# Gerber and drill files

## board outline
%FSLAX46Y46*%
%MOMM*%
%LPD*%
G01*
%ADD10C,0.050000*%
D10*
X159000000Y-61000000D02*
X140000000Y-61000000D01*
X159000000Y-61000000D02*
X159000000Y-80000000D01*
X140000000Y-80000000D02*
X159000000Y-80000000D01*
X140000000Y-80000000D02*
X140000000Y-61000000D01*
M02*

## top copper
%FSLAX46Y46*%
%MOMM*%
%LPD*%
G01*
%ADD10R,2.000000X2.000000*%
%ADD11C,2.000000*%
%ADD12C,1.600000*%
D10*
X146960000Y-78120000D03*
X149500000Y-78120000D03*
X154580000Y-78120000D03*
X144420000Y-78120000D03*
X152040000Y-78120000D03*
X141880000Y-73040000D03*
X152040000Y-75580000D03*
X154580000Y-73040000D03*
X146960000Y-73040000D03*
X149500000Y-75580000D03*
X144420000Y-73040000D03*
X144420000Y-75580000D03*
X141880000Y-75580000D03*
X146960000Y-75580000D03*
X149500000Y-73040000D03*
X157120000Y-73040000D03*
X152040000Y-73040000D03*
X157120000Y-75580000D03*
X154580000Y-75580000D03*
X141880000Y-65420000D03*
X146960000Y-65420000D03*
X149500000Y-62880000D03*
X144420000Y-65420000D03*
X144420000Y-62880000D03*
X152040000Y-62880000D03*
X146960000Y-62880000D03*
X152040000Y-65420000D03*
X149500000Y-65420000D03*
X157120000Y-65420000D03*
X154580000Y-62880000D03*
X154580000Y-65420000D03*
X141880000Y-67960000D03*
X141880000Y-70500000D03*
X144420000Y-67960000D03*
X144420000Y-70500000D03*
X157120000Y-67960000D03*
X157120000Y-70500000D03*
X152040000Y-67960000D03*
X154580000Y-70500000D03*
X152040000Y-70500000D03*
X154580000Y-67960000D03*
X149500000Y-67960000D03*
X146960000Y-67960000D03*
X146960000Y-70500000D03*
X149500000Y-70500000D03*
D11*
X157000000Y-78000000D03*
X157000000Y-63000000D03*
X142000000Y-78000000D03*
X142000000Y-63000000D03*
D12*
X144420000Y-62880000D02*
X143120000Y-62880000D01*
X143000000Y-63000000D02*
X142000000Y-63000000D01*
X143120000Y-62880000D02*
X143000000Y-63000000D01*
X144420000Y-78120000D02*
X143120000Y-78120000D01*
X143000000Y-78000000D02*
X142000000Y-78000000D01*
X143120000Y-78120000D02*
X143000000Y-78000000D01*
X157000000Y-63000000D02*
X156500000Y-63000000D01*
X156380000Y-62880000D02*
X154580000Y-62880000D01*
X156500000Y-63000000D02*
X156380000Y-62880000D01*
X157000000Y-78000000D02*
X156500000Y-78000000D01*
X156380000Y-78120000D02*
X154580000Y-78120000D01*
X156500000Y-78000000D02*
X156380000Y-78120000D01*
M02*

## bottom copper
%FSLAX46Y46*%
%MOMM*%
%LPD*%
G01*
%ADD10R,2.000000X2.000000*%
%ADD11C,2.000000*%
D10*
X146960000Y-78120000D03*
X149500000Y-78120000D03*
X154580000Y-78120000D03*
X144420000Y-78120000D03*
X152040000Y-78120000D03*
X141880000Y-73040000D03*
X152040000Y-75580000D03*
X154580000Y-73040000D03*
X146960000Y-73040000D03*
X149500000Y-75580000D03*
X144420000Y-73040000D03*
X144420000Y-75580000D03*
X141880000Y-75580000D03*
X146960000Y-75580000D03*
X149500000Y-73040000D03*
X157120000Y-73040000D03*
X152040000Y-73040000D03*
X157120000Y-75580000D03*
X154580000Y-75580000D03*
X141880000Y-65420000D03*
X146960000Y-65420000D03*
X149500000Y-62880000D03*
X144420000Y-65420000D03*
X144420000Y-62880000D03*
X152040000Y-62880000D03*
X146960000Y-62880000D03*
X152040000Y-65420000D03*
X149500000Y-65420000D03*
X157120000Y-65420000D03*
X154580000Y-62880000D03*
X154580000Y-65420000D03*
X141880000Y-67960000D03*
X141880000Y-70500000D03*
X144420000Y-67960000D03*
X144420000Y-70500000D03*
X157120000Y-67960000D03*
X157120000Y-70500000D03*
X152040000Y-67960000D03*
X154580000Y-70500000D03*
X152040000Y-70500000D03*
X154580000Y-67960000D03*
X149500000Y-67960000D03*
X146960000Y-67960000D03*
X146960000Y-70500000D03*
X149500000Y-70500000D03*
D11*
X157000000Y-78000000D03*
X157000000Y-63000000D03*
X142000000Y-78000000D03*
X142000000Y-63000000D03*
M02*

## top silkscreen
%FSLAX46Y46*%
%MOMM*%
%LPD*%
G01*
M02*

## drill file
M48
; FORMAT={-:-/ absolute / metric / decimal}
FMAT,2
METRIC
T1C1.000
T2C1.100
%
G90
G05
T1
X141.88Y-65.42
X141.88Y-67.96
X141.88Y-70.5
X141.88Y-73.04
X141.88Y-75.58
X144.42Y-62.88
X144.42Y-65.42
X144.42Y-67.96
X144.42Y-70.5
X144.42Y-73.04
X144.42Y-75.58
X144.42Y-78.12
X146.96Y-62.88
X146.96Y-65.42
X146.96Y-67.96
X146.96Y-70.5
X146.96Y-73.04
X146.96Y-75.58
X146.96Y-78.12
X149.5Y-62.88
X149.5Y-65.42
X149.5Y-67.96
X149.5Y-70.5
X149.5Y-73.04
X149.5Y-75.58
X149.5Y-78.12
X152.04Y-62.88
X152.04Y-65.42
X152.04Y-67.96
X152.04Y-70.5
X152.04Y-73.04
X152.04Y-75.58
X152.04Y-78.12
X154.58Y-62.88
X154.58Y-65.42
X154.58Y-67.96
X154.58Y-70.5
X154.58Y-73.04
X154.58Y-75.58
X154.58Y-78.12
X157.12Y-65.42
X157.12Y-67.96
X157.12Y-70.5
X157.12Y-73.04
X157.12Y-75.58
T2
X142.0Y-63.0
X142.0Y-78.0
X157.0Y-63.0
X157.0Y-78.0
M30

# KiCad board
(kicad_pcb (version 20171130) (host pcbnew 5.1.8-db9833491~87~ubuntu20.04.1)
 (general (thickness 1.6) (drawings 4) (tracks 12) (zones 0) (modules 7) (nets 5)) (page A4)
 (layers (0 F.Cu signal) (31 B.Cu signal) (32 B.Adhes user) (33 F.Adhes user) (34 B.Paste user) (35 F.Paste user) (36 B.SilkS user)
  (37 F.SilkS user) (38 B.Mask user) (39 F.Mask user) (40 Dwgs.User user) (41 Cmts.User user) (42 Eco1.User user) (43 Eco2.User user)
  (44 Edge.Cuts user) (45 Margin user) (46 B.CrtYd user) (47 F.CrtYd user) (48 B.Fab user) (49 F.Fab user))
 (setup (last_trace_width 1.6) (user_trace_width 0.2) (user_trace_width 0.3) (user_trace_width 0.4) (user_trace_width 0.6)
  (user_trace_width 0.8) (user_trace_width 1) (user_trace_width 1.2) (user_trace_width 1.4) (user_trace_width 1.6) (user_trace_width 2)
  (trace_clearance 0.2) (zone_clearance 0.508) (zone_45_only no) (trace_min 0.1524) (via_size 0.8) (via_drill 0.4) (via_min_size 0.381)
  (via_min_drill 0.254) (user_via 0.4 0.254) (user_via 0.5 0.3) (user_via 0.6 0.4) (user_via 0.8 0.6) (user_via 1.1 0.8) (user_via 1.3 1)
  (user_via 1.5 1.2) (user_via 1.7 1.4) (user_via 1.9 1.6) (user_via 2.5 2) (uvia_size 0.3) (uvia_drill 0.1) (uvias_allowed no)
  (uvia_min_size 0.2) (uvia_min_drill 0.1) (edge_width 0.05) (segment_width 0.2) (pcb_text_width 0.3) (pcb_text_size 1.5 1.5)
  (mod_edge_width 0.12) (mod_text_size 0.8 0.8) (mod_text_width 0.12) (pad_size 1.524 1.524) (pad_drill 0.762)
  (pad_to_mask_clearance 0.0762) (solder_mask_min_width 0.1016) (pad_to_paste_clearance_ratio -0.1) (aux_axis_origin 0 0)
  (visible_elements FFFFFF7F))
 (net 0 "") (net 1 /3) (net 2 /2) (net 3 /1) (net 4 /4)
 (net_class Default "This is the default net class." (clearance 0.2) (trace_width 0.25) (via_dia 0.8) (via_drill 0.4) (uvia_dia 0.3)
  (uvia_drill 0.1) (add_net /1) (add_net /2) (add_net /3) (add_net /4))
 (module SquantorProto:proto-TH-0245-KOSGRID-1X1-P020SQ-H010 (layer F.Cu) (at 149.5 70.5)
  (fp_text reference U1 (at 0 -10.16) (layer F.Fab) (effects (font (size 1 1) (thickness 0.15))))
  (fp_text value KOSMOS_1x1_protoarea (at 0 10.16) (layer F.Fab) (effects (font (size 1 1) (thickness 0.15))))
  (pad NC thru_hole rect (at -2.54 7.62) (size 2 2) (drill 1) (layers *.Cu *.Mask))
  (pad NC thru_hole rect (at 0 7.62) (size 2 2) (drill 1) (layers *.Cu *.Mask))
  (pad 3 thru_hole rect (at 5.08 7.62) (size 2 2) (drill 1) (layers *.Cu *.Mask) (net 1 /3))
  (pad 2 thru_hole rect (at -5.08 7.62) (size 2 2) (drill 1) (layers *.Cu *.Mask) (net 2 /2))
  (pad NC thru_hole rect (at 2.54 7.62) (size 2 2) (drill 1) (layers *.Cu *.Mask))
  (pad NC thru_hole rect (at -7.62 2.54) (size 2 2) (drill 1) (layers *.Cu *.Mask))
  (pad NC thru_hole rect (at 2.54 5.08) (size 2 2) (drill 1) (layers *.Cu *.Mask))
  (pad NC thru_hole rect (at 5.08 2.54) (size 2 2) (drill 1) (layers *.Cu *.Mask))
  (pad NC thru_hole rect (at -2.54 2.54) (size 2 2) (drill 1) (layers *.Cu *.Mask))
  (pad NC thru_hole rect (at 0 5.08) (size 2 2) (drill 1) (layers *.Cu *.Mask))
  (pad NC thru_hole rect (at -5.08 2.54) (size 2 2) (drill 1) (layers *.Cu *.Mask))
  (pad NC thru_hole rect (at -5.08 5.08) (size 2 2) (drill 1) (layers *.Cu *.Mask))
  (pad NC thru_hole rect (at -7.62 5.08) (size 2 2) (drill 1) (layers *.Cu *.Mask))
  (pad NC thru_hole rect (at -2.54 5.08) (size 2 2) (drill 1) (layers *.Cu *.Mask))
  (pad NC thru_hole rect (at 0 2.54) (size 2 2) (drill 1) (layers *.Cu *.Mask))
  (pad NC thru_hole rect (at 7.62 2.54) (size 2 2) (drill 1) (layers *.Cu *.Mask))
  (pad NC thru_hole rect (at 2.54 2.54) (size 2 2) (drill 1) (layers *.Cu *.Mask))
  (pad NC thru_hole rect (at 7.62 5.08) (size 2 2) (drill 1) (layers *.Cu *.Mask))
  (pad NC thru_hole rect (at 5.08 5.08) (size 2 2) (drill 1) (layers *.Cu *.Mask))
  (pad NC thru_hole rect (at -7.62 -5.08) (size 2 2) (drill 1) (layers *.Cu *.Mask))
  (pad NC thru_hole rect (at -2.54 -5.08) (size 2 2) (drill 1) (layers *.Cu *.Mask))
  (pad NC thru_hole rect (at 0 -7.62) (size 2 2) (drill 1) (layers *.Cu *.Mask))
  (pad NC thru_hole rect (at -5.08 -5.08) (size 2 2) (drill 1) (layers *.Cu *.Mask))
  (pad 1 thru_hole rect (at -5.08 -7.62) (size 2 2) (drill 1) (layers *.Cu *.Mask) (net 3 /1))
  (pad NC thru_hole rect (at 2.54 -7.62) (size 2 2) (drill 1) (layers *.Cu *.Mask))
  (pad NC thru_hole rect (at -2.54 -7.62) (size 2 2) (drill 1) (layers *.Cu *.Mask))
  (pad NC thru_hole rect (at 2.54 -5.08) (size 2 2) (drill 1) (layers *.Cu *.Mask))
  (pad NC thru_hole rect (at 0 -5.08) (size 2 2) (drill 1) (layers *.Cu *.Mask))
  (pad NC thru_hole rect (at 7.62 -5.08) (size 2 2) (drill 1) (layers *.Cu *.Mask))
  (pad 4 thru_hole rect (at 5.08 -7.62) (size 2 2) (drill 1) (layers *.Cu *.Mask) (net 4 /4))
  (pad NC thru_hole rect (at 5.08 -5.08) (size 2 2) (drill 1) (layers *.Cu *.Mask))
  (pad NC thru_hole rect (at -7.62 -2.54) (size 2 2) (drill 1) (layers *.Cu *.Mask))
  (pad NC thru_hole rect (at -7.62 0) (size 2 2) (drill 1) (layers *.Cu *.Mask))
  (pad NC thru_hole rect (at -5.08 -2.54) (size 2 2) (drill 1) (layers *.Cu *.Mask))
  (pad NC thru_hole rect (at -5.08 0) (size 2 2) (drill 1) (layers *.Cu *.Mask))
  (pad NC thru_hole rect (at 7.62 -2.54) (size 2 2) (drill 1) (layers *.Cu *.Mask))
  (pad NC thru_hole rect (at 7.62 0) (size 2 2) (drill 1) (layers *.Cu *.Mask))
  (pad NC thru_hole rect (at 2.54 -2.54) (size 2 2) (drill 1) (layers *.Cu *.Mask))
  (pad NC thru_hole rect (at 5.08 0) (size 2 2) (drill 1) (layers *.Cu *.Mask))
  (pad NC thru_hole rect (at 2.54 0) (size 2 2) (drill 1) (layers *.Cu *.Mask))
  (pad NC thru_hole rect (at 5.08 -2.54) (size 2 2) (drill 1) (layers *.Cu *.Mask))
  (pad NC thru_hole rect (at 0 -2.54) (size 2 2) (drill 1) (layers *.Cu *.Mask))
  (pad NC thru_hole rect (at -2.54 -2.54) (size 2 2) (drill 1) (layers *.Cu *.Mask))
  (pad NC thru_hole rect (at -2.54 0) (size 2 2) (drill 1) (layers *.Cu *.Mask))
  (pad NC thru_hole rect (at 0 0) (size 2 2) (drill 1) (layers *.Cu *.Mask)))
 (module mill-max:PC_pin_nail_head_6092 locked (layer F.Cu) (at 157 78)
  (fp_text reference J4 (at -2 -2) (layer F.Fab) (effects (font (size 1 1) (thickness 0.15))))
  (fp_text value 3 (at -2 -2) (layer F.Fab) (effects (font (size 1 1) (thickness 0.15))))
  (pad 1 thru_hole circle (at 0 0) (size 2 2) (drill 1.1) (layers *.Cu *.Mask) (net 1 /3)))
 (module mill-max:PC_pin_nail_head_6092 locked (layer F.Cu) (at 157 63)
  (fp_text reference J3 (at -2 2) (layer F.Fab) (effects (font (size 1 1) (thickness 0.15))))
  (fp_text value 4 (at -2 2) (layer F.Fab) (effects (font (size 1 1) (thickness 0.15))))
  (pad 1 thru_hole circle (at 0 0) (size 2 2) (drill 1.1) (layers *.Cu *.Mask) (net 4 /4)))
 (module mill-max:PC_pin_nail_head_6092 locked (layer F.Cu) (at 142 78)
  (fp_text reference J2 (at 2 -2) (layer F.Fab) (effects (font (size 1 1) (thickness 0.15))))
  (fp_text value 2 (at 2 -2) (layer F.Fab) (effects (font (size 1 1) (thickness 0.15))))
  (pad 1 thru_hole circle (at 0 0) (size 2 2) (drill 1.1) (layers *.Cu *.Mask) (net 2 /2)))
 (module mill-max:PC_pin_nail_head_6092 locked (layer F.Cu) (at 142 63)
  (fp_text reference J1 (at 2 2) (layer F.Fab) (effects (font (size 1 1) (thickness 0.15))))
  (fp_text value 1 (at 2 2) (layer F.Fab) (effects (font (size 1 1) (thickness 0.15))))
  (pad 1 thru_hole circle (at 0 0) (size 2 2) (drill 1.1) (layers *.Cu *.Mask) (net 3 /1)))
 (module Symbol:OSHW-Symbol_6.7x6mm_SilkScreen (layer B.Cu) (at 149.7 69.6 180)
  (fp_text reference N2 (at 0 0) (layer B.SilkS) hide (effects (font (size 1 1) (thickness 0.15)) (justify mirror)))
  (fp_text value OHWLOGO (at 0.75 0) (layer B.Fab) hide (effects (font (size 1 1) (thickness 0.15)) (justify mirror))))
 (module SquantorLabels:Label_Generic (layer B.Cu) (at 149.1 73.5)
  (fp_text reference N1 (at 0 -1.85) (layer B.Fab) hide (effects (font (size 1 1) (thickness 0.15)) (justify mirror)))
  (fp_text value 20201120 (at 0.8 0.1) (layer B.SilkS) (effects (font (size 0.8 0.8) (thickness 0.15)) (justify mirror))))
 (gr_line (start 159 61) (end 140 61) (layer Edge.Cuts) (width 0.05))
 (gr_line (start 159 61) (end 159 80) (layer Edge.Cuts) (width 0.05))
 (gr_line (start 140 80) (end 159 80) (layer Edge.Cuts) (width 0.05))
 (gr_line (start 140 80) (end 140 61) (layer Edge.Cuts) (width 0.05))
 (segment (start 144.42 62.88) (end 143.12 62.88) (width 1.6) (layer F.Cu) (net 3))
 (segment (start 143 63) (end 142 63) (width 1.6) (layer F.Cu) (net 3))
 (segment (start 143.12 62.88) (end 143 63) (width 1.6) (layer F.Cu) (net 3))
 (segment (start 144.42 78.12) (end 143.12 78.12) (width 1.6) (layer F.Cu) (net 2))
 (segment (start 143 78) (end 142 78) (width 1.6) (layer F.Cu) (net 2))
 (segment (start 143.12 78.12) (end 143 78) (width 1.6) (layer F.Cu) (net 2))
 (segment (start 157 63) (end 156.5 63) (width 1.6) (layer F.Cu) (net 4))
 (segment (start 156.38 62.88) (end 154.58 62.88) (width 1.6) (layer F.Cu) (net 4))
 (segment (start 156.5 63) (end 156.38 62.88) (width 1.6) (layer F.Cu) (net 4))
 (segment (start 157 78) (end 156.5 78) (width 1.6) (layer F.Cu) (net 1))
 (segment (start 156.38 78.12) (end 154.58 78.12) (width 1.6) (layer F.Cu) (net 1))
 (segment (start 156.5 78) (end 156.38 78.12) (width 1.6) (layer F.Cu) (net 1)))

